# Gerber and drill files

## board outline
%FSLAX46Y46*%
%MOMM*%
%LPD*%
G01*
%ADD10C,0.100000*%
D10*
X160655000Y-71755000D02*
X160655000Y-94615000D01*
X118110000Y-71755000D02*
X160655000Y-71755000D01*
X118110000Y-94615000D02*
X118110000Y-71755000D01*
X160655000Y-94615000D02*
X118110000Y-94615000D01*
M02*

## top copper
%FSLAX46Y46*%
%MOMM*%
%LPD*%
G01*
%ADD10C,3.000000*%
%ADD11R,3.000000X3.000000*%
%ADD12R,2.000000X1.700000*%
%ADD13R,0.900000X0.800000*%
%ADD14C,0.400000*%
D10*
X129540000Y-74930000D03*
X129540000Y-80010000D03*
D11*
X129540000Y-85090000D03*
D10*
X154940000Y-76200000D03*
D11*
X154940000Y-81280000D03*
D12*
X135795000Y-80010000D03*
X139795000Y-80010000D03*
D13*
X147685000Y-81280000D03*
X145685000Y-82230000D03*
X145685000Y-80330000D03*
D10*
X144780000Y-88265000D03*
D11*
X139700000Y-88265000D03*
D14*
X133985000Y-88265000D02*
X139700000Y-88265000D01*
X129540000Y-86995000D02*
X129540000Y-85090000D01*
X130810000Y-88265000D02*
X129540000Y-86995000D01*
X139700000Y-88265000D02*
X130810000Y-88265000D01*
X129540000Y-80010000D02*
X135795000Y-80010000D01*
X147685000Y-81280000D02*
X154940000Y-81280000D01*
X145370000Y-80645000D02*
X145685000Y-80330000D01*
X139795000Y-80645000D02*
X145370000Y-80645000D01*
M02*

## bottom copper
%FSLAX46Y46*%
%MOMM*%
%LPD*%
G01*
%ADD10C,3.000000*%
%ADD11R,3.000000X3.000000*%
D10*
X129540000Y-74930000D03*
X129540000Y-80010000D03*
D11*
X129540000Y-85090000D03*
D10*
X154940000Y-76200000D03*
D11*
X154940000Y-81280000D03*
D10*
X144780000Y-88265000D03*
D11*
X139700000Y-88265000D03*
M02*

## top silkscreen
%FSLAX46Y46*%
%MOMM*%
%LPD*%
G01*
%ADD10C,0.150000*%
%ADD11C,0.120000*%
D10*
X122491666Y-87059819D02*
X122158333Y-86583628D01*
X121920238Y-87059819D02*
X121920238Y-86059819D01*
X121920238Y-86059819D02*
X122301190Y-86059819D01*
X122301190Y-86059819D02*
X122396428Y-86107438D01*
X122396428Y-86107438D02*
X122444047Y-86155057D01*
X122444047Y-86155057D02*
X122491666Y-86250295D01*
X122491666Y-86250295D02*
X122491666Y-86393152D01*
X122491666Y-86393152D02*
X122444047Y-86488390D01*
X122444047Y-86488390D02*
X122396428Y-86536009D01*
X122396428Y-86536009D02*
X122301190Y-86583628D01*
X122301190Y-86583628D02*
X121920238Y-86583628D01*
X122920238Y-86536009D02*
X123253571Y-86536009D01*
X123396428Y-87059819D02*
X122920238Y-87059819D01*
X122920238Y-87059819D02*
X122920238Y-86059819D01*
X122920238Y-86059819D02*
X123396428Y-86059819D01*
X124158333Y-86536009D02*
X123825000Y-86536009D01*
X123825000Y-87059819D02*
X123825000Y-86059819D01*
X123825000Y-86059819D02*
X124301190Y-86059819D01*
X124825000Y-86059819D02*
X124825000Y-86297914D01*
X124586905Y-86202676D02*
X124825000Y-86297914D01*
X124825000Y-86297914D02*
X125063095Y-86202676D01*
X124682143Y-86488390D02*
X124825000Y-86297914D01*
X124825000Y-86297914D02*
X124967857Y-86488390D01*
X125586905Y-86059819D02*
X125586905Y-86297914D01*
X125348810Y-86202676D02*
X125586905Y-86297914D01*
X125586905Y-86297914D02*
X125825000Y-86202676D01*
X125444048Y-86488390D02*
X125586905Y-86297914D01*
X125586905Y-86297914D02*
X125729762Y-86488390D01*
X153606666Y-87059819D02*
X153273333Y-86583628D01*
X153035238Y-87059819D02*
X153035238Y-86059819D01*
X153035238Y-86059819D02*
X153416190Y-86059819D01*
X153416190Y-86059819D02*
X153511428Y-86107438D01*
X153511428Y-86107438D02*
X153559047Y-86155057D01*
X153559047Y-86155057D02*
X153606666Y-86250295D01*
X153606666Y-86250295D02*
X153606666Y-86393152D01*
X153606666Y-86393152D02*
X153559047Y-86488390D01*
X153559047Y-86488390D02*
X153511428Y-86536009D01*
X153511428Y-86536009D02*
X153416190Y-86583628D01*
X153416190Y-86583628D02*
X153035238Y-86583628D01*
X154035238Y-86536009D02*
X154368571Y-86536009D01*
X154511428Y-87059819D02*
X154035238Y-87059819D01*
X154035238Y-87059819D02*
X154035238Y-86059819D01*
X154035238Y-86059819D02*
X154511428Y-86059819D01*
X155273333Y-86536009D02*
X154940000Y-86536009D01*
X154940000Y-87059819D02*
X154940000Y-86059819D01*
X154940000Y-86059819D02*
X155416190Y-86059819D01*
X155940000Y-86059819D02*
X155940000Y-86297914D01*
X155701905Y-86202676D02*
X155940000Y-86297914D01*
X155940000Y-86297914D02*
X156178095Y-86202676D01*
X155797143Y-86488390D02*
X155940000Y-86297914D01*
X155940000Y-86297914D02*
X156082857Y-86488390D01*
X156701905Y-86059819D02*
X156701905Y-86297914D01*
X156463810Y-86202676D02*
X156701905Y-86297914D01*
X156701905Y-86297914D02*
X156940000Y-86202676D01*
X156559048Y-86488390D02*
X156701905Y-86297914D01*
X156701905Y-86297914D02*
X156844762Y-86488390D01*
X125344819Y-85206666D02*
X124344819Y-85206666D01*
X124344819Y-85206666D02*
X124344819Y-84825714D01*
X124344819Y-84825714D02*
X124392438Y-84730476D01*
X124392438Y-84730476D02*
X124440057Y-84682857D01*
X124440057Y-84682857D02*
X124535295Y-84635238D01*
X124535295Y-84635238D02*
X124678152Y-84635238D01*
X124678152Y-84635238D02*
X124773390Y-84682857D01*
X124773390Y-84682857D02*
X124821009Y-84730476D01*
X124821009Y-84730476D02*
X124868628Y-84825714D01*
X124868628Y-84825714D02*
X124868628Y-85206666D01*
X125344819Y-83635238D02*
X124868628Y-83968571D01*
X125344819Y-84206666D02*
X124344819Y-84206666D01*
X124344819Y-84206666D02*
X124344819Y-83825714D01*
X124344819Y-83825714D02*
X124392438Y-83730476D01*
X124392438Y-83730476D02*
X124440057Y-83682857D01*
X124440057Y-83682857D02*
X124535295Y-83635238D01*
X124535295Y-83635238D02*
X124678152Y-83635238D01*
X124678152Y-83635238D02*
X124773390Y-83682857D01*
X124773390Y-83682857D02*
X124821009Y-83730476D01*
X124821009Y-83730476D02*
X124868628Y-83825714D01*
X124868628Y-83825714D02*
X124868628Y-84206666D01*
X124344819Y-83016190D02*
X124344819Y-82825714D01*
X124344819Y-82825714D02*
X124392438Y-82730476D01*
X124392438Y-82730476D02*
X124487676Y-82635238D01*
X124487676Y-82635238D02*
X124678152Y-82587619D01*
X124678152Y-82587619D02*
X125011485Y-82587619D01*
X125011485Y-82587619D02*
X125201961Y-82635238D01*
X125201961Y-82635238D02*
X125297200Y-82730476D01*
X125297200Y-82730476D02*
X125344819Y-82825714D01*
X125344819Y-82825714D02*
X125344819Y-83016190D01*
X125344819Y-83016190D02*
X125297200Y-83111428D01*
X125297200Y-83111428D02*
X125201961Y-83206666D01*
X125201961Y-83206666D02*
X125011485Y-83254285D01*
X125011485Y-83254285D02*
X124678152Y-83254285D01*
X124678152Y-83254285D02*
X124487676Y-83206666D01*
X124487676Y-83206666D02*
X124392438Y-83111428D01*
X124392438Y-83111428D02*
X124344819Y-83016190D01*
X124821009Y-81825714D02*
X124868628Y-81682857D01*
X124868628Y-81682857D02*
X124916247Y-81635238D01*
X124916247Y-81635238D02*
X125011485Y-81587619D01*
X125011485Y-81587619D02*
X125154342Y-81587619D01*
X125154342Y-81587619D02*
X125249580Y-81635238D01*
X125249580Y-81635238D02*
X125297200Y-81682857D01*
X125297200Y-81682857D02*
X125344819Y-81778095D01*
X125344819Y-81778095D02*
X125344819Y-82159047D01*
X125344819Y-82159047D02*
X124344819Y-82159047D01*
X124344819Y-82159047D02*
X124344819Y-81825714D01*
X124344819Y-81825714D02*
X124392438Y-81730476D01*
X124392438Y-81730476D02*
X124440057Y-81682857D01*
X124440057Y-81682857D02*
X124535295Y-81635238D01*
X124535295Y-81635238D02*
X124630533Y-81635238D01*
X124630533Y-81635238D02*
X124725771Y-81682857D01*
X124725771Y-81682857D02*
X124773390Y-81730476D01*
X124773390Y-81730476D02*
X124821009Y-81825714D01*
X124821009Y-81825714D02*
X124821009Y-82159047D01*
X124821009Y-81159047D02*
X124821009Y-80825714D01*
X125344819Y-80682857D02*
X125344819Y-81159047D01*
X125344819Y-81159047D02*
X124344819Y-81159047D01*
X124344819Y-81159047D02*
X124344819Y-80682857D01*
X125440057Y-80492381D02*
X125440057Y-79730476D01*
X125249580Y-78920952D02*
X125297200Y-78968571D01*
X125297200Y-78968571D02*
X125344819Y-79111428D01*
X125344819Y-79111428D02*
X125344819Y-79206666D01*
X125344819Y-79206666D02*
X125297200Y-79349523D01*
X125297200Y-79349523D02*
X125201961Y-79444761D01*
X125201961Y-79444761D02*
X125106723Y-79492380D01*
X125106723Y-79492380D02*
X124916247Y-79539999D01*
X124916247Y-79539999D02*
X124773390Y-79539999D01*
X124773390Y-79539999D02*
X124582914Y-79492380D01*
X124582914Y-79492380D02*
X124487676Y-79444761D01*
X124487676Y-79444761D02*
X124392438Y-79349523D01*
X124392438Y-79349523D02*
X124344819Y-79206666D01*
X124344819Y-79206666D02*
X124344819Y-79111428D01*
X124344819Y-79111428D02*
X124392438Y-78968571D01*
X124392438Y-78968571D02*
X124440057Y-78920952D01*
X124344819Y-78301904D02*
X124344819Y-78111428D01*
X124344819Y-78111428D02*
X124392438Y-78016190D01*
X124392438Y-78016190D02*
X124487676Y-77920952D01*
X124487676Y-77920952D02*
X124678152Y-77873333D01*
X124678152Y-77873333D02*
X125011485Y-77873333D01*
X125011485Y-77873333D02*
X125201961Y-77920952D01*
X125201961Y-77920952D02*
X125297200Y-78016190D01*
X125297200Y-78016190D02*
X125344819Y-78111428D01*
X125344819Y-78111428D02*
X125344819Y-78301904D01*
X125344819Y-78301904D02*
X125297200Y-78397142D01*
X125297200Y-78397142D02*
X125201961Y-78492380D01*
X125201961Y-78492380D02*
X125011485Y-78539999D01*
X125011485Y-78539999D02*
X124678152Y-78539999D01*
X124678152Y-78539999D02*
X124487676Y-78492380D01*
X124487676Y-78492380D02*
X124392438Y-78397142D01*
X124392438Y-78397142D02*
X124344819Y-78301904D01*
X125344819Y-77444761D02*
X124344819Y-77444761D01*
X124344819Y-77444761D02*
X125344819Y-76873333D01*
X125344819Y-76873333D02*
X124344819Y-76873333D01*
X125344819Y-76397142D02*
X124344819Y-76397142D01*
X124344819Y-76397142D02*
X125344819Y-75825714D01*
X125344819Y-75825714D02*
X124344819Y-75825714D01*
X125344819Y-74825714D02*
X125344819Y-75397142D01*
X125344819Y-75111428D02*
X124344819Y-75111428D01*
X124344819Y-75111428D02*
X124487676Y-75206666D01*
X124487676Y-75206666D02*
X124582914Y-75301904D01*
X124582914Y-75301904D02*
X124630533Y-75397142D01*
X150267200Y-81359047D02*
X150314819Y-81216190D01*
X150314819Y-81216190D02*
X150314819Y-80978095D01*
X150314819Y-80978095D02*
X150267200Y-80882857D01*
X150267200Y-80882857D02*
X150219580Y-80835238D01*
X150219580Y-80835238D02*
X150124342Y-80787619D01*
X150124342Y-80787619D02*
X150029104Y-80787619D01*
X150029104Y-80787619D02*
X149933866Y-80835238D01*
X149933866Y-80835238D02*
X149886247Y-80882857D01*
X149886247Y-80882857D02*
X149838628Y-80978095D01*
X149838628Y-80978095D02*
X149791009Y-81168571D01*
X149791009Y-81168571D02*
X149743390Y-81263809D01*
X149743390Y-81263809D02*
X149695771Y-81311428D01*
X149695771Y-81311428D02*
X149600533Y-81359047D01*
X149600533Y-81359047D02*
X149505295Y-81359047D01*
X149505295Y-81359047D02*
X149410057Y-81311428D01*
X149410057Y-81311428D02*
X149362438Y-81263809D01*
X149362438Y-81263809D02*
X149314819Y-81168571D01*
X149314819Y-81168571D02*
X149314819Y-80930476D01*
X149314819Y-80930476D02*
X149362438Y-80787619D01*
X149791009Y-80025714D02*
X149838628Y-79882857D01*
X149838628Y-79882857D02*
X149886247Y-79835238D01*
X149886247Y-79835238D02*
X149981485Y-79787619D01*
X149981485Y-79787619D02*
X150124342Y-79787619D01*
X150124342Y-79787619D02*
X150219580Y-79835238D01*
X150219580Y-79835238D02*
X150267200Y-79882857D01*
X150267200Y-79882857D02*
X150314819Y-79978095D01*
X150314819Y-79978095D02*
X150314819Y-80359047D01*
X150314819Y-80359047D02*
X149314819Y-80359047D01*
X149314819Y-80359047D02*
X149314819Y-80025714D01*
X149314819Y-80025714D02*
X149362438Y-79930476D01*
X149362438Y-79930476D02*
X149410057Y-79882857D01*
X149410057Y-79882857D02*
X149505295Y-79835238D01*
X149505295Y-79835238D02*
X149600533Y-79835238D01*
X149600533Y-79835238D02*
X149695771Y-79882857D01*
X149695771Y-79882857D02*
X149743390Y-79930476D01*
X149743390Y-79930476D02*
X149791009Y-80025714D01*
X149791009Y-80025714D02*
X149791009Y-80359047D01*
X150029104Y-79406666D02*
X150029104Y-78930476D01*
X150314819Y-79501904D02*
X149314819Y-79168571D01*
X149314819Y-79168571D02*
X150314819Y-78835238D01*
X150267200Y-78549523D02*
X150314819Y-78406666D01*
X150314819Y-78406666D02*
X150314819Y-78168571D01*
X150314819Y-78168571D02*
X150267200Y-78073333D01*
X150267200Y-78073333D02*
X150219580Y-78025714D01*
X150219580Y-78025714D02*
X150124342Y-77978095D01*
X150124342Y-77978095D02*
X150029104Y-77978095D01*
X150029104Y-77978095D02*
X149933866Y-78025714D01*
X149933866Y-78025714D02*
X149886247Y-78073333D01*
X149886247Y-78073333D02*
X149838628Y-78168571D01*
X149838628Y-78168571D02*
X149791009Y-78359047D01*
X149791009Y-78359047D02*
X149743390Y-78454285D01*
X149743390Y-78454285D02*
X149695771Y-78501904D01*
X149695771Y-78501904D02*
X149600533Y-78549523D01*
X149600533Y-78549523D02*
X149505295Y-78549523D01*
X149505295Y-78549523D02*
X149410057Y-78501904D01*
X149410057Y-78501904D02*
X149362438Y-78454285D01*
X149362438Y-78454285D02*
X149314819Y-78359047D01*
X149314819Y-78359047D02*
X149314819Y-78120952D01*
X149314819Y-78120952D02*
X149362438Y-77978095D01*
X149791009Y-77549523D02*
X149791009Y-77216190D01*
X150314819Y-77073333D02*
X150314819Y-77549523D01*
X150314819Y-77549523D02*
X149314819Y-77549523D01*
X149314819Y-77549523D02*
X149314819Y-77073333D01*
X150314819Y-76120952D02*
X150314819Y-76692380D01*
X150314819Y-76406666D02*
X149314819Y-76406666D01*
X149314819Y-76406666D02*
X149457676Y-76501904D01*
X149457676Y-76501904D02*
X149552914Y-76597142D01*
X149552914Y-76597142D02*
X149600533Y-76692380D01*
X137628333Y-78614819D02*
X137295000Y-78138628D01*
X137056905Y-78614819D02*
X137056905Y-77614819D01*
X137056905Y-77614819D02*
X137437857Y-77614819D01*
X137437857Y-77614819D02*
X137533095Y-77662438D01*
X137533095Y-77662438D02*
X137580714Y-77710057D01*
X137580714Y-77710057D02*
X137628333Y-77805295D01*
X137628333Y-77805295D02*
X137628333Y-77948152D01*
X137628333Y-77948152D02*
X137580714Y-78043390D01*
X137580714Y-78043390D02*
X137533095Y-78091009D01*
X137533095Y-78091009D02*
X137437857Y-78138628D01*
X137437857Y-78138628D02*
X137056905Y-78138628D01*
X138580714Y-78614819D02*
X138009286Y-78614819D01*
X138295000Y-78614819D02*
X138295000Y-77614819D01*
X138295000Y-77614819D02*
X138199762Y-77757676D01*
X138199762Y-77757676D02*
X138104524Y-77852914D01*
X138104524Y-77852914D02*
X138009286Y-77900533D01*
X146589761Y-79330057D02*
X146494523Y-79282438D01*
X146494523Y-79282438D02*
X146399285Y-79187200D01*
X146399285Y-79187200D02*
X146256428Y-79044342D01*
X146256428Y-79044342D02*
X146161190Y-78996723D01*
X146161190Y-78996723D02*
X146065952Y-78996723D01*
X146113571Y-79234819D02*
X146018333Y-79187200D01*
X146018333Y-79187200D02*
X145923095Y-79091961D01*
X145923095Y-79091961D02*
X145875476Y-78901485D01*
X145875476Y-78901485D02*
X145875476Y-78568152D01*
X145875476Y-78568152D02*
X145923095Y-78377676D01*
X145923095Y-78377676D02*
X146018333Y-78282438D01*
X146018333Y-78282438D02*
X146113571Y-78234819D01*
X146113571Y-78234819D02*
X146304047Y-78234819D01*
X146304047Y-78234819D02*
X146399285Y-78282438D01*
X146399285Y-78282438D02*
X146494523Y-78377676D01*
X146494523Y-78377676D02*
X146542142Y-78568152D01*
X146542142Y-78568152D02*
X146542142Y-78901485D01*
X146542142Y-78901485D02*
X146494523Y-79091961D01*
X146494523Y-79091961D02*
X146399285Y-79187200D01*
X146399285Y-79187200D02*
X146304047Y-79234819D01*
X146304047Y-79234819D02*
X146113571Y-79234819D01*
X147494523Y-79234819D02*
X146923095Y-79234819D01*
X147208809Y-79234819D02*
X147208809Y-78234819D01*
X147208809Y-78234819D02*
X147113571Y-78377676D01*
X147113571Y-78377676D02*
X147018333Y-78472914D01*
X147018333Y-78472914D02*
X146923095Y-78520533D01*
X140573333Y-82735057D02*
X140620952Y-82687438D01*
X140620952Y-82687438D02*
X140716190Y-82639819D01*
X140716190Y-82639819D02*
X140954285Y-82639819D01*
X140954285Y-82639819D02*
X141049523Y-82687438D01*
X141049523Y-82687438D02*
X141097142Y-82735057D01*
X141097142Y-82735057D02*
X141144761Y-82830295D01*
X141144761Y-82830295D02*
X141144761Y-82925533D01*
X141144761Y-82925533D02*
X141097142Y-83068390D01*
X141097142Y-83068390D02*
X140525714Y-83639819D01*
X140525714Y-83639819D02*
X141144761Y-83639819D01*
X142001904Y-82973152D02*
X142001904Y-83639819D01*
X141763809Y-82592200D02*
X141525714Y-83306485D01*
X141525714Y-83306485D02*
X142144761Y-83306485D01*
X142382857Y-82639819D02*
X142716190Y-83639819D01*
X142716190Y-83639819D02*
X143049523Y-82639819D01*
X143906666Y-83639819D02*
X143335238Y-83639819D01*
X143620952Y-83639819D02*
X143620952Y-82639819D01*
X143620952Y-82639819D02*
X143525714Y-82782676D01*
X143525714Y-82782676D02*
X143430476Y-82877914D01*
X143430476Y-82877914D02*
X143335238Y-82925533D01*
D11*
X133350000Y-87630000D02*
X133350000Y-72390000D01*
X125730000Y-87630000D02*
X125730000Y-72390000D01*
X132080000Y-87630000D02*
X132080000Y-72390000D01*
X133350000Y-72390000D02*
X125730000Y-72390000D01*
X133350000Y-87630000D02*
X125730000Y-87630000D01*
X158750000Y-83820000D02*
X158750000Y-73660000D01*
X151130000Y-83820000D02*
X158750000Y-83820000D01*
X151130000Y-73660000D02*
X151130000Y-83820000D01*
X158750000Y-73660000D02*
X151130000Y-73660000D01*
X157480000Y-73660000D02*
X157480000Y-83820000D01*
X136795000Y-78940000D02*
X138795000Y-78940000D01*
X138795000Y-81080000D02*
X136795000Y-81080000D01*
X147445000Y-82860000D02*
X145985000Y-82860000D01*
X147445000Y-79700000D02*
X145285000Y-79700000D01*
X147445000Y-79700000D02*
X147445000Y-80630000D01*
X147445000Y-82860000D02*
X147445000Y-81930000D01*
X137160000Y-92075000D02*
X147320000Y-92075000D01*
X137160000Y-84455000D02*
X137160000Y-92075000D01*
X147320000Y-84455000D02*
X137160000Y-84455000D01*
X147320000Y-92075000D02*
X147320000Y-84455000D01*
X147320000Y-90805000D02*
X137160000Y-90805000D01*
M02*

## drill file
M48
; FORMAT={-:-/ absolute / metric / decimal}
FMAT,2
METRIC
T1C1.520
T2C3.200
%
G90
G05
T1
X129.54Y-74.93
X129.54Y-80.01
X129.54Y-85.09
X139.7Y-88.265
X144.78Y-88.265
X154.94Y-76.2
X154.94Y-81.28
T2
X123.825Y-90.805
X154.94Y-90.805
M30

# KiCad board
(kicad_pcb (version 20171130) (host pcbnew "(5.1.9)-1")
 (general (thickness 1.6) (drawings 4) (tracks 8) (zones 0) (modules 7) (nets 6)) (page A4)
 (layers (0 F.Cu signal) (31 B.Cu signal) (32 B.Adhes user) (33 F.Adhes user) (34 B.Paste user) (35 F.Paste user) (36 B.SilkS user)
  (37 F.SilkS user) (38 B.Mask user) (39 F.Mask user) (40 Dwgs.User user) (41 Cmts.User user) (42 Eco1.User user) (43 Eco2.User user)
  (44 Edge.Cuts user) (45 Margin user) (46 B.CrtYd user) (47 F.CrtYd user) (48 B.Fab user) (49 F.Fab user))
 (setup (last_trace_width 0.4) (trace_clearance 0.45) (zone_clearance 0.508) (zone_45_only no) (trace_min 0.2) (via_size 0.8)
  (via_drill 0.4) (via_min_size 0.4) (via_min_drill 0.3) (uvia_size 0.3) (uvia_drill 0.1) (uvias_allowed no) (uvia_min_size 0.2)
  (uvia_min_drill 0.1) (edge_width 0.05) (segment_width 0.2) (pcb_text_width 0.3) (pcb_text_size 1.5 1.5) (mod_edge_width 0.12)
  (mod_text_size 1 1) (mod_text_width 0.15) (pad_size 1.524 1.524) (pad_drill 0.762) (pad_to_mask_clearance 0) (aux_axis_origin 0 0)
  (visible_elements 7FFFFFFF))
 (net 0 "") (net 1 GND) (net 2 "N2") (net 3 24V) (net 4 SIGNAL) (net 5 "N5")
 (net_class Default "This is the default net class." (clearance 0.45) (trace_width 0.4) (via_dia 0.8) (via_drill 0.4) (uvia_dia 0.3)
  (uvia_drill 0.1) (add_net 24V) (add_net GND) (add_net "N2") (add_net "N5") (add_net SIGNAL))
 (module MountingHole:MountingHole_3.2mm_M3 (layer F.Cu) (at 123.825 90.805)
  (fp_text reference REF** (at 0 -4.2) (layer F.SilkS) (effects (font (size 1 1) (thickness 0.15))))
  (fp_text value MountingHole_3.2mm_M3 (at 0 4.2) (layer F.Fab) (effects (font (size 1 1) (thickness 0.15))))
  (pad 1 np_thru_hole circle (at 0 0) (size 3.2 3.2) (drill 3.2) (layers *.Cu *.Mask)))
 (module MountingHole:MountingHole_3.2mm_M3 (layer F.Cu) (at 154.94 90.805)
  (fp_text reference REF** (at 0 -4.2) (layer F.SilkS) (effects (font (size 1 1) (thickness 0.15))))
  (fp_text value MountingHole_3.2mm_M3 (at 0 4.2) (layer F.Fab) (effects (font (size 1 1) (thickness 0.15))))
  (pad 1 np_thru_hole circle (at 0 0) (size 3.2 3.2) (drill 3.2) (layers *.Cu *.Mask)))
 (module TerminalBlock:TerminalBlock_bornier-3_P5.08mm (layer F.Cu) (at 129.54 85.09 90)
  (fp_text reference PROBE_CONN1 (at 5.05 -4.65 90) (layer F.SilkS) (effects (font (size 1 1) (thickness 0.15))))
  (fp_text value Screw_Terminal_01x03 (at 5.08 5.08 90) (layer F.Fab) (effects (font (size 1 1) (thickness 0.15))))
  (fp_line (start -2.54 3.81) (end 12.7 3.81) (layer F.SilkS) (width 0.12))
  (fp_line (start -2.54 -3.81) (end 12.7 -3.81) (layer F.SilkS) (width 0.12))
  (fp_line (start -2.54 2.54) (end 12.7 2.54) (layer F.SilkS) (width 0.12))
  (fp_line (start 12.7 3.81) (end 12.7 -3.81) (layer F.SilkS) (width 0.12))
  (fp_line (start -2.54 3.81) (end -2.54 -3.81) (layer F.SilkS) (width 0.12))
  (pad 3 thru_hole circle (at 10.16 0 90) (size 3 3) (drill 1.52) (layers *.Cu *.Mask) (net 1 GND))
  (pad 2 thru_hole circle (at 5.08 0 90) (size 3 3) (drill 1.52) (layers *.Cu *.Mask) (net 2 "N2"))
  (pad 1 thru_hole rect (at 0 0 90) (size 3 3) (drill 1.52) (layers *.Cu *.Mask) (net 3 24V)))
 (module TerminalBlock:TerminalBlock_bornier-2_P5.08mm (layer F.Cu) (at 154.94 81.28 90)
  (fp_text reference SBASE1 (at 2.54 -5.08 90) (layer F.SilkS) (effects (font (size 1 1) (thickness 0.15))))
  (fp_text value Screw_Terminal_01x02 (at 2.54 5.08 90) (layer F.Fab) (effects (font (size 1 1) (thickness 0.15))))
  (fp_line (start -2.54 3.81) (end 7.62 3.81) (layer F.SilkS) (width 0.12))
  (fp_line (start -2.54 -3.81) (end -2.54 3.81) (layer F.SilkS) (width 0.12))
  (fp_line (start 7.62 -3.81) (end -2.54 -3.81) (layer F.SilkS) (width 0.12))
  (fp_line (start 7.62 3.81) (end 7.62 -3.81) (layer F.SilkS) (width 0.12))
  (fp_line (start 7.62 2.54) (end -2.54 2.54) (layer F.SilkS) (width 0.12))
  (pad 2 thru_hole circle (at 5.08 0 90) (size 3 3) (drill 1.52) (layers *.Cu *.Mask) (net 1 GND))
  (pad 1 thru_hole rect (at 0 0 90) (size 3 3) (drill 1.52) (layers *.Cu *.Mask) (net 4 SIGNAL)))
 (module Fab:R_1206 (layer F.Cu) (at 137.795 80.01)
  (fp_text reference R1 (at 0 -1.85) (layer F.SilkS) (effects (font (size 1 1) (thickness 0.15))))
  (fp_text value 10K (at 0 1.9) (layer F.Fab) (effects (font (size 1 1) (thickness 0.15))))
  (fp_line (start -1 -1.07) (end 1 -1.07) (layer F.SilkS) (width 0.12))
  (fp_line (start 1 1.07) (end -1 1.07) (layer F.SilkS) (width 0.12))
  (pad 1 smd rect (at -2 0) (size 2 1.7) (layers F.Cu F.Paste F.Mask) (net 2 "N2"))
  (pad 2 smd rect (at 2 0) (size 2 1.7) (layers F.Cu F.Paste F.Mask) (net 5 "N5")))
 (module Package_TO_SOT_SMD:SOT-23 (layer F.Cu) (at 146.685 81.28)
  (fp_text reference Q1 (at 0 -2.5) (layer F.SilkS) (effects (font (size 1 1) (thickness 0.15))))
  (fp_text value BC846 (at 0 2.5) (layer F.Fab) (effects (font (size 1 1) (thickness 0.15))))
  (fp_line (start 0.76 1.58) (end -0.7 1.58) (layer F.SilkS) (width 0.12))
  (fp_line (start 0.76 -1.58) (end -1.4 -1.58) (layer F.SilkS) (width 0.12))
  (fp_line (start 0.76 -1.58) (end 0.76 -0.65) (layer F.SilkS) (width 0.12))
  (fp_line (start 0.76 1.58) (end 0.76 0.65) (layer F.SilkS) (width 0.12))
  (pad 3 smd rect (at 1 0) (size 0.9 0.8) (layers F.Cu F.Paste F.Mask) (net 4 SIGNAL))
  (pad 2 smd rect (at -1 0.95) (size 0.9 0.8) (layers F.Cu F.Paste F.Mask) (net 1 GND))
  (pad 1 smd rect (at -1 -0.95) (size 0.9 0.8) (layers F.Cu F.Paste F.Mask) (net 5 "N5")))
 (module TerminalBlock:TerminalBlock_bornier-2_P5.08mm (layer F.Cu) (at 139.7 88.265)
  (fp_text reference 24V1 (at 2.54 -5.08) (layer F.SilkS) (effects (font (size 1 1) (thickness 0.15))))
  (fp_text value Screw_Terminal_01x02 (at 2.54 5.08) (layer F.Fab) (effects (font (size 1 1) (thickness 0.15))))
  (fp_line (start -2.54 3.81) (end 7.62 3.81) (layer F.SilkS) (width 0.12))
  (fp_line (start -2.54 -3.81) (end -2.54 3.81) (layer F.SilkS) (width 0.12))
  (fp_line (start 7.62 -3.81) (end -2.54 -3.81) (layer F.SilkS) (width 0.12))
  (fp_line (start 7.62 3.81) (end 7.62 -3.81) (layer F.SilkS) (width 0.12))
  (fp_line (start 7.62 2.54) (end -2.54 2.54) (layer F.SilkS) (width 0.12))
  (pad 2 thru_hole circle (at 5.08 0) (size 3 3) (drill 1.52) (layers *.Cu *.Mask) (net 1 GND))
  (pad 1 thru_hole rect (at 0 0) (size 3 3) (drill 1.52) (layers *.Cu *.Mask) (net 3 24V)))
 (gr_line (start 160.655 71.755) (end 160.655 94.615) (layer Edge.Cuts) (width 0.1))
 (gr_line (start 118.11 71.755) (end 160.655 71.755) (layer Edge.Cuts) (width 0.1))
 (gr_line (start 118.11 94.615) (end 118.11 71.755) (layer Edge.Cuts) (width 0.1))
 (gr_line (start 160.655 94.615) (end 118.11 94.615) (layer Edge.Cuts) (width 0.1))
 (segment (start 133.985 88.265) (end 139.7 88.265) (width 0.4) (layer F.Cu) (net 3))
 (segment (start 129.54 86.995) (end 129.54 85.09) (width 0.4) (layer F.Cu) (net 3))
 (segment (start 130.81 88.265) (end 129.54 86.995) (width 0.4) (layer F.Cu) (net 3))
 (segment (start 139.7 88.265) (end 130.81 88.265) (width 0.4) (layer F.Cu) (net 3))
 (segment (start 129.54 80.01) (end 135.795 80.01) (width 0.4) (layer F.Cu) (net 2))
 (segment (start 147.685 81.28) (end 154.94 81.28) (width 0.4) (layer F.Cu) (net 4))
 (segment (start 145.37 80.645) (end 145.685 80.33) (width 0.4) (layer F.Cu) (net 5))
 (segment (start 139.795 80.645) (end 145.37 80.645) (width 0.4) (layer F.Cu) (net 5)))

